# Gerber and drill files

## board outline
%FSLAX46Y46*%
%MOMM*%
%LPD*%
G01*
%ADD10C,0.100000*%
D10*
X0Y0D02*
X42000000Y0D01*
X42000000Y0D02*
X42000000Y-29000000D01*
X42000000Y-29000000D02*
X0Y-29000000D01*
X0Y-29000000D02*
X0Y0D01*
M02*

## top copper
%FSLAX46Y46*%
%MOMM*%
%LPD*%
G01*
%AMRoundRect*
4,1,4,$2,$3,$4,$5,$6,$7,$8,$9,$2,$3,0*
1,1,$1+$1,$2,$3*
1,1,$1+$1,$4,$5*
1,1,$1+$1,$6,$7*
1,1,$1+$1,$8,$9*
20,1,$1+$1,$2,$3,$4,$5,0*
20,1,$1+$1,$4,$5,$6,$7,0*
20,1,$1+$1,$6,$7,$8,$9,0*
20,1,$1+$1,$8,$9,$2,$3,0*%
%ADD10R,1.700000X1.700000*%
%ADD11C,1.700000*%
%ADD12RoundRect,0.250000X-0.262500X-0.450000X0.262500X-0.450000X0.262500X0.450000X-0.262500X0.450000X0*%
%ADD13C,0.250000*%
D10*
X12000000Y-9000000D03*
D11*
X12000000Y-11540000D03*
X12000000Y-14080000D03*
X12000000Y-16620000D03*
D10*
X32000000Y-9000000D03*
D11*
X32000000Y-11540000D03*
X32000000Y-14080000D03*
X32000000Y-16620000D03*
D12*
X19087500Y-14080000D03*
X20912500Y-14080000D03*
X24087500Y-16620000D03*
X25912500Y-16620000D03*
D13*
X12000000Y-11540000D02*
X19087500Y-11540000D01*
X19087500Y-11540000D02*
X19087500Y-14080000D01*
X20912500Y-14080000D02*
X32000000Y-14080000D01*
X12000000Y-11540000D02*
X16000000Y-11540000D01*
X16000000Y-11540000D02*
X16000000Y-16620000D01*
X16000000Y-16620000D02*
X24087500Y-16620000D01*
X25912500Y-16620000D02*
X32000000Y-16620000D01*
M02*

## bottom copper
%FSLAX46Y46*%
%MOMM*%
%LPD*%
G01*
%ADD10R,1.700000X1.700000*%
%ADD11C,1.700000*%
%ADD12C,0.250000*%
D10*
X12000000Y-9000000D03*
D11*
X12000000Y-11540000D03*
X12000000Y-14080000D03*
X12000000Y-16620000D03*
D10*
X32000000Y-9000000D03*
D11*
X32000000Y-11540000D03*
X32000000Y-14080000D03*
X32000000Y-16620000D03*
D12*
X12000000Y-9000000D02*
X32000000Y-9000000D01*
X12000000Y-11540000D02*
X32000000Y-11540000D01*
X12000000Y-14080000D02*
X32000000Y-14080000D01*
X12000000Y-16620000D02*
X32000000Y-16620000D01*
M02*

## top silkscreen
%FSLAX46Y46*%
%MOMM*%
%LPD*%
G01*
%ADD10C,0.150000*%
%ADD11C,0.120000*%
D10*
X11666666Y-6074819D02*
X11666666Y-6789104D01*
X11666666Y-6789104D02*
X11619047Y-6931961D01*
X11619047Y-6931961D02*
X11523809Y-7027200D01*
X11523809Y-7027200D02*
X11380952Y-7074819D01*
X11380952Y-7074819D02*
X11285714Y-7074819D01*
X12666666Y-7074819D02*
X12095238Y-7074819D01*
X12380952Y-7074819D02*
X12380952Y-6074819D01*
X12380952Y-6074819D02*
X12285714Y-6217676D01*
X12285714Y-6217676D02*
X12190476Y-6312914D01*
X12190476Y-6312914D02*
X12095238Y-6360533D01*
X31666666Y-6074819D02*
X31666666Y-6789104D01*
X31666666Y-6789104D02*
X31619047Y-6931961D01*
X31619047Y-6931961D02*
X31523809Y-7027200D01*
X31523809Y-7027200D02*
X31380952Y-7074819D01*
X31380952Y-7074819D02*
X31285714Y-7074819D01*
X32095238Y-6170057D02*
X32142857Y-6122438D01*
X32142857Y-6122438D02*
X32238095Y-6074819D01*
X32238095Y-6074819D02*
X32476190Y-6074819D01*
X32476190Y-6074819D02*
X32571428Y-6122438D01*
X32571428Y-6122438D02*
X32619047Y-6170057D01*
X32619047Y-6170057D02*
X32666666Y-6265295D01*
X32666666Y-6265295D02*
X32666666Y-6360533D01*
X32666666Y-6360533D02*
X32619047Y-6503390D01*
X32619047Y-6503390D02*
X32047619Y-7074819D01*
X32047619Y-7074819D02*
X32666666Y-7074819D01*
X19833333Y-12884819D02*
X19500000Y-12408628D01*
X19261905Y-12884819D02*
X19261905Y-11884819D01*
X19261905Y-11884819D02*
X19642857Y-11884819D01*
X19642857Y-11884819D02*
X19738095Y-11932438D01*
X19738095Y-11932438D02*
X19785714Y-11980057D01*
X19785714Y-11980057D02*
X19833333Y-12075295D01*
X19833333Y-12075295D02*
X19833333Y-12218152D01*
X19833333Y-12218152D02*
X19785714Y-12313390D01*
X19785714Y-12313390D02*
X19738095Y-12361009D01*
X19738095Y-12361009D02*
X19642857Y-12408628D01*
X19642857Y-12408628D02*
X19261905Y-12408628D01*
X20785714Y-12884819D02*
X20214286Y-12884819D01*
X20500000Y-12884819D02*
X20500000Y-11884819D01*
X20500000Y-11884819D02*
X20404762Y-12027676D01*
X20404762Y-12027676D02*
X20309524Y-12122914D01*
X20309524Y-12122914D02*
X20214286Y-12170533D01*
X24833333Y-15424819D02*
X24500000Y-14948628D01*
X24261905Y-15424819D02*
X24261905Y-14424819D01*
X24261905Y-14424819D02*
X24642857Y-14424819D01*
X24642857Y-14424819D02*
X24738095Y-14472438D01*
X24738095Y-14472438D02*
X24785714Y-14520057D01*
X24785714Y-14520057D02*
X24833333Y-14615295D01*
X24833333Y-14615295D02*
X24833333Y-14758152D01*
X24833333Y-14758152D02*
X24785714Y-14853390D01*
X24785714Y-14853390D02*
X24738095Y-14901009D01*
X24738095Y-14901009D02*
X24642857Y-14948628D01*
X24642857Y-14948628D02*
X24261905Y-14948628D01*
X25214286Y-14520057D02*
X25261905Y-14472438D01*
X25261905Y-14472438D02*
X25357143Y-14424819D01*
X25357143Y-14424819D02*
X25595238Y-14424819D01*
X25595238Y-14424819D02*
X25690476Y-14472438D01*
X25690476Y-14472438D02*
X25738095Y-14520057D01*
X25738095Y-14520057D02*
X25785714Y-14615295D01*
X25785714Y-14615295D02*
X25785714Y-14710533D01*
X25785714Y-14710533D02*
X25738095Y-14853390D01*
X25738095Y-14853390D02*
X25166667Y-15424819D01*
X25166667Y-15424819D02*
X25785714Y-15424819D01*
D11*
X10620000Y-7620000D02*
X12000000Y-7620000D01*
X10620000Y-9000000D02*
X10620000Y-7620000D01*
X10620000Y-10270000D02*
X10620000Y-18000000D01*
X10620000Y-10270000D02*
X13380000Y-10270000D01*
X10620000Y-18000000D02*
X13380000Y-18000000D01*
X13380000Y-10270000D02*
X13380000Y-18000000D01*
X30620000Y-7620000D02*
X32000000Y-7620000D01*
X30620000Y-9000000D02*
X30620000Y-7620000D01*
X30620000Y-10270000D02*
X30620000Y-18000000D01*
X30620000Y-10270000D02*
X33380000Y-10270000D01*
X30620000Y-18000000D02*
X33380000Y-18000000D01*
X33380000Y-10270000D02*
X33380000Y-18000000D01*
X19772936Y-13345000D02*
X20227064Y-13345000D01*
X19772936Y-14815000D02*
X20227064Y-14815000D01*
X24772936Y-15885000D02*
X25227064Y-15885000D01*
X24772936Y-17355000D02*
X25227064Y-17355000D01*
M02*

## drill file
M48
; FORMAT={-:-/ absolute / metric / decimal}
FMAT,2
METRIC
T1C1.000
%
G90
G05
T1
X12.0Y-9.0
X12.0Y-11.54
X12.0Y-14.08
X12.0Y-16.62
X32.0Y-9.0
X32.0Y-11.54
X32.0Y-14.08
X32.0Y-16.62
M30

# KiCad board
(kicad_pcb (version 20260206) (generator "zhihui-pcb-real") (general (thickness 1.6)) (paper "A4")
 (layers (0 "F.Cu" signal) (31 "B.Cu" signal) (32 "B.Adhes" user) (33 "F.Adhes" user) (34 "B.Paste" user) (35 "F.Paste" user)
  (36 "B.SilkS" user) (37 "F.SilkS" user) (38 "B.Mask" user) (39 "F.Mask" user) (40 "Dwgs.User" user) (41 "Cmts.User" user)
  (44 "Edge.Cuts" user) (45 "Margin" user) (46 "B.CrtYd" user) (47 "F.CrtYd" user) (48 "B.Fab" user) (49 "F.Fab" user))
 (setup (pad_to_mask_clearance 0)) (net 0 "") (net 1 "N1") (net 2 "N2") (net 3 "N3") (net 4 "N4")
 (gr_line (start 0 0) (end 42 0) (stroke (width 0.1) (type default)) (layer "Edge.Cuts"))
 (gr_line (start 42 0) (end 42 29) (stroke (width 0.1) (type default)) (layer "Edge.Cuts"))
 (gr_line (start 42 29) (end 0 29) (stroke (width 0.1) (type default)) (layer "Edge.Cuts"))
 (gr_line (start 0 29) (end 0 0) (stroke (width 0.1) (type default)) (layer "Edge.Cuts"))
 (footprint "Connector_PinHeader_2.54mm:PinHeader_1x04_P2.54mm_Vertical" (layer "F.Cu")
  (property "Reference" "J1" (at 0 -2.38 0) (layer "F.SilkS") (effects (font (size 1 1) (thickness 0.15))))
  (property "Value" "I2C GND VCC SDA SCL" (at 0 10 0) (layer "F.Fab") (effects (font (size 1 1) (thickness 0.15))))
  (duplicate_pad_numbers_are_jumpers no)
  (fp_line (start -1.38 -1.38) (end 0 -1.38) (stroke (width 0.12) (type solid)) (layer "F.SilkS"))
  (fp_line (start -1.38 0) (end -1.38 -1.38) (stroke (width 0.12) (type solid)) (layer "F.SilkS"))
  (fp_line (start -1.38 1.27) (end -1.38 9) (stroke (width 0.12) (type solid)) (layer "F.SilkS"))
  (fp_line (start -1.38 1.27) (end 1.38 1.27) (stroke (width 0.12) (type solid)) (layer "F.SilkS"))
  (fp_line (start -1.38 9) (end 1.38 9) (stroke (width 0.12) (type solid)) (layer "F.SilkS"))
  (fp_line (start 1.38 1.27) (end 1.38 9) (stroke (width 0.12) (type solid)) (layer "F.SilkS"))
  (pad "1" thru_hole rect (at 0 0) (size 1.7 1.7) (drill 1) (layers "*.Cu" "*.Mask") (remove_unused_layers no) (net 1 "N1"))
  (pad "2" thru_hole circle (at 0 2.54) (size 1.7 1.7) (drill 1) (layers "*.Cu" "*.Mask") (remove_unused_layers no) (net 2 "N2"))
  (pad "3" thru_hole circle (at 0 5.08) (size 1.7 1.7) (drill 1) (layers "*.Cu" "*.Mask") (remove_unused_layers no) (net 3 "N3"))
  (pad "4" thru_hole circle (at 0 7.62) (size 1.7 1.7) (drill 1) (layers "*.Cu" "*.Mask") (remove_unused_layers no) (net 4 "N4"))
  (at 12 9 0))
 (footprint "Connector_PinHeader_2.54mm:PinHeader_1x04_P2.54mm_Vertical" (layer "F.Cu")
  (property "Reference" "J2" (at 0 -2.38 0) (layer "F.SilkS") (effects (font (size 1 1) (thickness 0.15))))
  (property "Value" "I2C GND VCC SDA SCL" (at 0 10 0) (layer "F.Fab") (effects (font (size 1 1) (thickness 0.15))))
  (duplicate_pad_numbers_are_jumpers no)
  (fp_line (start -1.38 -1.38) (end 0 -1.38) (stroke (width 0.12) (type solid)) (layer "F.SilkS"))
  (fp_line (start -1.38 0) (end -1.38 -1.38) (stroke (width 0.12) (type solid)) (layer "F.SilkS"))
  (fp_line (start -1.38 1.27) (end -1.38 9) (stroke (width 0.12) (type solid)) (layer "F.SilkS"))
  (fp_line (start -1.38 1.27) (end 1.38 1.27) (stroke (width 0.12) (type solid)) (layer "F.SilkS"))
  (fp_line (start -1.38 9) (end 1.38 9) (stroke (width 0.12) (type solid)) (layer "F.SilkS"))
  (fp_line (start 1.38 1.27) (end 1.38 9) (stroke (width 0.12) (type solid)) (layer "F.SilkS"))
  (pad "1" thru_hole rect (at 0 0) (size 1.7 1.7) (drill 1) (layers "*.Cu" "*.Mask") (remove_unused_layers no) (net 1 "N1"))
  (pad "2" thru_hole circle (at 0 2.54) (size 1.7 1.7) (drill 1) (layers "*.Cu" "*.Mask") (remove_unused_layers no) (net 2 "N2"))
  (pad "3" thru_hole circle (at 0 5.08) (size 1.7 1.7) (drill 1) (layers "*.Cu" "*.Mask") (remove_unused_layers no) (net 3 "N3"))
  (pad "4" thru_hole circle (at 0 7.62) (size 1.7 1.7) (drill 1) (layers "*.Cu" "*.Mask") (remove_unused_layers no) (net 4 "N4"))
  (at 32 9 0))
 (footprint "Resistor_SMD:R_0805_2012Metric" (layer "F.Cu")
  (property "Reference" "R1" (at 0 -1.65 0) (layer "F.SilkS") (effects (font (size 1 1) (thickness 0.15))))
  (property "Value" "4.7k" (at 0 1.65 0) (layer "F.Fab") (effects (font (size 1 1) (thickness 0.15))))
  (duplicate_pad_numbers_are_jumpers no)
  (fp_line (start -0.227064 -0.735) (end 0.227064 -0.735) (stroke (width 0.12) (type solid)) (layer "F.SilkS"))
  (fp_line (start -0.227064 0.735) (end 0.227064 0.735) (stroke (width 0.12) (type solid)) (layer "F.SilkS"))
  (pad "1" smd roundrect (at -0.9125 0) (size 1.025 1.4) (layers "F.Cu" "F.Mask" "F.Paste") (roundrect_rratio 0.243902) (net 2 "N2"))
  (pad "2" smd roundrect (at 0.9125 0) (size 1.025 1.4) (layers "F.Cu" "F.Mask" "F.Paste") (roundrect_rratio 0.243902) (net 3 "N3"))
  (at 20 14.08 0))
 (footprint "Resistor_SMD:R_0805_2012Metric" (layer "F.Cu")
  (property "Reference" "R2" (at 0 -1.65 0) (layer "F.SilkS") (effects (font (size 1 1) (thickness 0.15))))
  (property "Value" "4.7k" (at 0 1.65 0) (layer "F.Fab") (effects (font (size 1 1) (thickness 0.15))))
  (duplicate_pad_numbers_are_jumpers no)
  (fp_line (start -0.227064 -0.735) (end 0.227064 -0.735) (stroke (width 0.12) (type solid)) (layer "F.SilkS"))
  (fp_line (start -0.227064 0.735) (end 0.227064 0.735) (stroke (width 0.12) (type solid)) (layer "F.SilkS"))
  (pad "1" smd roundrect (at -0.9125 0) (size 1.025 1.4) (layers "F.Cu" "F.Mask" "F.Paste") (roundrect_rratio 0.243902) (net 2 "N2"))
  (pad "2" smd roundrect (at 0.9125 0) (size 1.025 1.4) (layers "F.Cu" "F.Mask" "F.Paste") (roundrect_rratio 0.243902) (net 4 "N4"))
  (at 25 16.62 0))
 (segment (start 12 9) (end 32 9) (width 0.25) (layer "B.Cu") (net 1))
 (segment (start 12 11.54) (end 32 11.54) (width 0.25) (layer "B.Cu") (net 2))
 (segment (start 12 14.08) (end 32 14.08) (width 0.25) (layer "B.Cu") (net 3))
 (segment (start 12 16.62) (end 32 16.62) (width 0.25) (layer "B.Cu") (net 4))
 (segment (start 12 11.54) (end 19.0875 11.54) (width 0.25) (layer "F.Cu") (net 2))
 (segment (start 19.0875 11.54) (end 19.0875 14.08) (width 0.25) (layer "F.Cu") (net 2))
 (segment (start 20.9125 14.08) (end 32 14.08) (width 0.25) (layer "F.Cu") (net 3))
 (segment (start 12 11.54) (end 16 11.54) (width 0.25) (layer "F.Cu") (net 2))
 (segment (start 16 11.54) (end 16 16.62) (width 0.25) (layer "F.Cu") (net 2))
 (segment (start 16 16.62) (end 24.0875 16.62) (width 0.25) (layer "F.Cu") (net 2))
 (segment (start 25.9125 16.62) (end 32 16.62) (width 0.25) (layer "F.Cu") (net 4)))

